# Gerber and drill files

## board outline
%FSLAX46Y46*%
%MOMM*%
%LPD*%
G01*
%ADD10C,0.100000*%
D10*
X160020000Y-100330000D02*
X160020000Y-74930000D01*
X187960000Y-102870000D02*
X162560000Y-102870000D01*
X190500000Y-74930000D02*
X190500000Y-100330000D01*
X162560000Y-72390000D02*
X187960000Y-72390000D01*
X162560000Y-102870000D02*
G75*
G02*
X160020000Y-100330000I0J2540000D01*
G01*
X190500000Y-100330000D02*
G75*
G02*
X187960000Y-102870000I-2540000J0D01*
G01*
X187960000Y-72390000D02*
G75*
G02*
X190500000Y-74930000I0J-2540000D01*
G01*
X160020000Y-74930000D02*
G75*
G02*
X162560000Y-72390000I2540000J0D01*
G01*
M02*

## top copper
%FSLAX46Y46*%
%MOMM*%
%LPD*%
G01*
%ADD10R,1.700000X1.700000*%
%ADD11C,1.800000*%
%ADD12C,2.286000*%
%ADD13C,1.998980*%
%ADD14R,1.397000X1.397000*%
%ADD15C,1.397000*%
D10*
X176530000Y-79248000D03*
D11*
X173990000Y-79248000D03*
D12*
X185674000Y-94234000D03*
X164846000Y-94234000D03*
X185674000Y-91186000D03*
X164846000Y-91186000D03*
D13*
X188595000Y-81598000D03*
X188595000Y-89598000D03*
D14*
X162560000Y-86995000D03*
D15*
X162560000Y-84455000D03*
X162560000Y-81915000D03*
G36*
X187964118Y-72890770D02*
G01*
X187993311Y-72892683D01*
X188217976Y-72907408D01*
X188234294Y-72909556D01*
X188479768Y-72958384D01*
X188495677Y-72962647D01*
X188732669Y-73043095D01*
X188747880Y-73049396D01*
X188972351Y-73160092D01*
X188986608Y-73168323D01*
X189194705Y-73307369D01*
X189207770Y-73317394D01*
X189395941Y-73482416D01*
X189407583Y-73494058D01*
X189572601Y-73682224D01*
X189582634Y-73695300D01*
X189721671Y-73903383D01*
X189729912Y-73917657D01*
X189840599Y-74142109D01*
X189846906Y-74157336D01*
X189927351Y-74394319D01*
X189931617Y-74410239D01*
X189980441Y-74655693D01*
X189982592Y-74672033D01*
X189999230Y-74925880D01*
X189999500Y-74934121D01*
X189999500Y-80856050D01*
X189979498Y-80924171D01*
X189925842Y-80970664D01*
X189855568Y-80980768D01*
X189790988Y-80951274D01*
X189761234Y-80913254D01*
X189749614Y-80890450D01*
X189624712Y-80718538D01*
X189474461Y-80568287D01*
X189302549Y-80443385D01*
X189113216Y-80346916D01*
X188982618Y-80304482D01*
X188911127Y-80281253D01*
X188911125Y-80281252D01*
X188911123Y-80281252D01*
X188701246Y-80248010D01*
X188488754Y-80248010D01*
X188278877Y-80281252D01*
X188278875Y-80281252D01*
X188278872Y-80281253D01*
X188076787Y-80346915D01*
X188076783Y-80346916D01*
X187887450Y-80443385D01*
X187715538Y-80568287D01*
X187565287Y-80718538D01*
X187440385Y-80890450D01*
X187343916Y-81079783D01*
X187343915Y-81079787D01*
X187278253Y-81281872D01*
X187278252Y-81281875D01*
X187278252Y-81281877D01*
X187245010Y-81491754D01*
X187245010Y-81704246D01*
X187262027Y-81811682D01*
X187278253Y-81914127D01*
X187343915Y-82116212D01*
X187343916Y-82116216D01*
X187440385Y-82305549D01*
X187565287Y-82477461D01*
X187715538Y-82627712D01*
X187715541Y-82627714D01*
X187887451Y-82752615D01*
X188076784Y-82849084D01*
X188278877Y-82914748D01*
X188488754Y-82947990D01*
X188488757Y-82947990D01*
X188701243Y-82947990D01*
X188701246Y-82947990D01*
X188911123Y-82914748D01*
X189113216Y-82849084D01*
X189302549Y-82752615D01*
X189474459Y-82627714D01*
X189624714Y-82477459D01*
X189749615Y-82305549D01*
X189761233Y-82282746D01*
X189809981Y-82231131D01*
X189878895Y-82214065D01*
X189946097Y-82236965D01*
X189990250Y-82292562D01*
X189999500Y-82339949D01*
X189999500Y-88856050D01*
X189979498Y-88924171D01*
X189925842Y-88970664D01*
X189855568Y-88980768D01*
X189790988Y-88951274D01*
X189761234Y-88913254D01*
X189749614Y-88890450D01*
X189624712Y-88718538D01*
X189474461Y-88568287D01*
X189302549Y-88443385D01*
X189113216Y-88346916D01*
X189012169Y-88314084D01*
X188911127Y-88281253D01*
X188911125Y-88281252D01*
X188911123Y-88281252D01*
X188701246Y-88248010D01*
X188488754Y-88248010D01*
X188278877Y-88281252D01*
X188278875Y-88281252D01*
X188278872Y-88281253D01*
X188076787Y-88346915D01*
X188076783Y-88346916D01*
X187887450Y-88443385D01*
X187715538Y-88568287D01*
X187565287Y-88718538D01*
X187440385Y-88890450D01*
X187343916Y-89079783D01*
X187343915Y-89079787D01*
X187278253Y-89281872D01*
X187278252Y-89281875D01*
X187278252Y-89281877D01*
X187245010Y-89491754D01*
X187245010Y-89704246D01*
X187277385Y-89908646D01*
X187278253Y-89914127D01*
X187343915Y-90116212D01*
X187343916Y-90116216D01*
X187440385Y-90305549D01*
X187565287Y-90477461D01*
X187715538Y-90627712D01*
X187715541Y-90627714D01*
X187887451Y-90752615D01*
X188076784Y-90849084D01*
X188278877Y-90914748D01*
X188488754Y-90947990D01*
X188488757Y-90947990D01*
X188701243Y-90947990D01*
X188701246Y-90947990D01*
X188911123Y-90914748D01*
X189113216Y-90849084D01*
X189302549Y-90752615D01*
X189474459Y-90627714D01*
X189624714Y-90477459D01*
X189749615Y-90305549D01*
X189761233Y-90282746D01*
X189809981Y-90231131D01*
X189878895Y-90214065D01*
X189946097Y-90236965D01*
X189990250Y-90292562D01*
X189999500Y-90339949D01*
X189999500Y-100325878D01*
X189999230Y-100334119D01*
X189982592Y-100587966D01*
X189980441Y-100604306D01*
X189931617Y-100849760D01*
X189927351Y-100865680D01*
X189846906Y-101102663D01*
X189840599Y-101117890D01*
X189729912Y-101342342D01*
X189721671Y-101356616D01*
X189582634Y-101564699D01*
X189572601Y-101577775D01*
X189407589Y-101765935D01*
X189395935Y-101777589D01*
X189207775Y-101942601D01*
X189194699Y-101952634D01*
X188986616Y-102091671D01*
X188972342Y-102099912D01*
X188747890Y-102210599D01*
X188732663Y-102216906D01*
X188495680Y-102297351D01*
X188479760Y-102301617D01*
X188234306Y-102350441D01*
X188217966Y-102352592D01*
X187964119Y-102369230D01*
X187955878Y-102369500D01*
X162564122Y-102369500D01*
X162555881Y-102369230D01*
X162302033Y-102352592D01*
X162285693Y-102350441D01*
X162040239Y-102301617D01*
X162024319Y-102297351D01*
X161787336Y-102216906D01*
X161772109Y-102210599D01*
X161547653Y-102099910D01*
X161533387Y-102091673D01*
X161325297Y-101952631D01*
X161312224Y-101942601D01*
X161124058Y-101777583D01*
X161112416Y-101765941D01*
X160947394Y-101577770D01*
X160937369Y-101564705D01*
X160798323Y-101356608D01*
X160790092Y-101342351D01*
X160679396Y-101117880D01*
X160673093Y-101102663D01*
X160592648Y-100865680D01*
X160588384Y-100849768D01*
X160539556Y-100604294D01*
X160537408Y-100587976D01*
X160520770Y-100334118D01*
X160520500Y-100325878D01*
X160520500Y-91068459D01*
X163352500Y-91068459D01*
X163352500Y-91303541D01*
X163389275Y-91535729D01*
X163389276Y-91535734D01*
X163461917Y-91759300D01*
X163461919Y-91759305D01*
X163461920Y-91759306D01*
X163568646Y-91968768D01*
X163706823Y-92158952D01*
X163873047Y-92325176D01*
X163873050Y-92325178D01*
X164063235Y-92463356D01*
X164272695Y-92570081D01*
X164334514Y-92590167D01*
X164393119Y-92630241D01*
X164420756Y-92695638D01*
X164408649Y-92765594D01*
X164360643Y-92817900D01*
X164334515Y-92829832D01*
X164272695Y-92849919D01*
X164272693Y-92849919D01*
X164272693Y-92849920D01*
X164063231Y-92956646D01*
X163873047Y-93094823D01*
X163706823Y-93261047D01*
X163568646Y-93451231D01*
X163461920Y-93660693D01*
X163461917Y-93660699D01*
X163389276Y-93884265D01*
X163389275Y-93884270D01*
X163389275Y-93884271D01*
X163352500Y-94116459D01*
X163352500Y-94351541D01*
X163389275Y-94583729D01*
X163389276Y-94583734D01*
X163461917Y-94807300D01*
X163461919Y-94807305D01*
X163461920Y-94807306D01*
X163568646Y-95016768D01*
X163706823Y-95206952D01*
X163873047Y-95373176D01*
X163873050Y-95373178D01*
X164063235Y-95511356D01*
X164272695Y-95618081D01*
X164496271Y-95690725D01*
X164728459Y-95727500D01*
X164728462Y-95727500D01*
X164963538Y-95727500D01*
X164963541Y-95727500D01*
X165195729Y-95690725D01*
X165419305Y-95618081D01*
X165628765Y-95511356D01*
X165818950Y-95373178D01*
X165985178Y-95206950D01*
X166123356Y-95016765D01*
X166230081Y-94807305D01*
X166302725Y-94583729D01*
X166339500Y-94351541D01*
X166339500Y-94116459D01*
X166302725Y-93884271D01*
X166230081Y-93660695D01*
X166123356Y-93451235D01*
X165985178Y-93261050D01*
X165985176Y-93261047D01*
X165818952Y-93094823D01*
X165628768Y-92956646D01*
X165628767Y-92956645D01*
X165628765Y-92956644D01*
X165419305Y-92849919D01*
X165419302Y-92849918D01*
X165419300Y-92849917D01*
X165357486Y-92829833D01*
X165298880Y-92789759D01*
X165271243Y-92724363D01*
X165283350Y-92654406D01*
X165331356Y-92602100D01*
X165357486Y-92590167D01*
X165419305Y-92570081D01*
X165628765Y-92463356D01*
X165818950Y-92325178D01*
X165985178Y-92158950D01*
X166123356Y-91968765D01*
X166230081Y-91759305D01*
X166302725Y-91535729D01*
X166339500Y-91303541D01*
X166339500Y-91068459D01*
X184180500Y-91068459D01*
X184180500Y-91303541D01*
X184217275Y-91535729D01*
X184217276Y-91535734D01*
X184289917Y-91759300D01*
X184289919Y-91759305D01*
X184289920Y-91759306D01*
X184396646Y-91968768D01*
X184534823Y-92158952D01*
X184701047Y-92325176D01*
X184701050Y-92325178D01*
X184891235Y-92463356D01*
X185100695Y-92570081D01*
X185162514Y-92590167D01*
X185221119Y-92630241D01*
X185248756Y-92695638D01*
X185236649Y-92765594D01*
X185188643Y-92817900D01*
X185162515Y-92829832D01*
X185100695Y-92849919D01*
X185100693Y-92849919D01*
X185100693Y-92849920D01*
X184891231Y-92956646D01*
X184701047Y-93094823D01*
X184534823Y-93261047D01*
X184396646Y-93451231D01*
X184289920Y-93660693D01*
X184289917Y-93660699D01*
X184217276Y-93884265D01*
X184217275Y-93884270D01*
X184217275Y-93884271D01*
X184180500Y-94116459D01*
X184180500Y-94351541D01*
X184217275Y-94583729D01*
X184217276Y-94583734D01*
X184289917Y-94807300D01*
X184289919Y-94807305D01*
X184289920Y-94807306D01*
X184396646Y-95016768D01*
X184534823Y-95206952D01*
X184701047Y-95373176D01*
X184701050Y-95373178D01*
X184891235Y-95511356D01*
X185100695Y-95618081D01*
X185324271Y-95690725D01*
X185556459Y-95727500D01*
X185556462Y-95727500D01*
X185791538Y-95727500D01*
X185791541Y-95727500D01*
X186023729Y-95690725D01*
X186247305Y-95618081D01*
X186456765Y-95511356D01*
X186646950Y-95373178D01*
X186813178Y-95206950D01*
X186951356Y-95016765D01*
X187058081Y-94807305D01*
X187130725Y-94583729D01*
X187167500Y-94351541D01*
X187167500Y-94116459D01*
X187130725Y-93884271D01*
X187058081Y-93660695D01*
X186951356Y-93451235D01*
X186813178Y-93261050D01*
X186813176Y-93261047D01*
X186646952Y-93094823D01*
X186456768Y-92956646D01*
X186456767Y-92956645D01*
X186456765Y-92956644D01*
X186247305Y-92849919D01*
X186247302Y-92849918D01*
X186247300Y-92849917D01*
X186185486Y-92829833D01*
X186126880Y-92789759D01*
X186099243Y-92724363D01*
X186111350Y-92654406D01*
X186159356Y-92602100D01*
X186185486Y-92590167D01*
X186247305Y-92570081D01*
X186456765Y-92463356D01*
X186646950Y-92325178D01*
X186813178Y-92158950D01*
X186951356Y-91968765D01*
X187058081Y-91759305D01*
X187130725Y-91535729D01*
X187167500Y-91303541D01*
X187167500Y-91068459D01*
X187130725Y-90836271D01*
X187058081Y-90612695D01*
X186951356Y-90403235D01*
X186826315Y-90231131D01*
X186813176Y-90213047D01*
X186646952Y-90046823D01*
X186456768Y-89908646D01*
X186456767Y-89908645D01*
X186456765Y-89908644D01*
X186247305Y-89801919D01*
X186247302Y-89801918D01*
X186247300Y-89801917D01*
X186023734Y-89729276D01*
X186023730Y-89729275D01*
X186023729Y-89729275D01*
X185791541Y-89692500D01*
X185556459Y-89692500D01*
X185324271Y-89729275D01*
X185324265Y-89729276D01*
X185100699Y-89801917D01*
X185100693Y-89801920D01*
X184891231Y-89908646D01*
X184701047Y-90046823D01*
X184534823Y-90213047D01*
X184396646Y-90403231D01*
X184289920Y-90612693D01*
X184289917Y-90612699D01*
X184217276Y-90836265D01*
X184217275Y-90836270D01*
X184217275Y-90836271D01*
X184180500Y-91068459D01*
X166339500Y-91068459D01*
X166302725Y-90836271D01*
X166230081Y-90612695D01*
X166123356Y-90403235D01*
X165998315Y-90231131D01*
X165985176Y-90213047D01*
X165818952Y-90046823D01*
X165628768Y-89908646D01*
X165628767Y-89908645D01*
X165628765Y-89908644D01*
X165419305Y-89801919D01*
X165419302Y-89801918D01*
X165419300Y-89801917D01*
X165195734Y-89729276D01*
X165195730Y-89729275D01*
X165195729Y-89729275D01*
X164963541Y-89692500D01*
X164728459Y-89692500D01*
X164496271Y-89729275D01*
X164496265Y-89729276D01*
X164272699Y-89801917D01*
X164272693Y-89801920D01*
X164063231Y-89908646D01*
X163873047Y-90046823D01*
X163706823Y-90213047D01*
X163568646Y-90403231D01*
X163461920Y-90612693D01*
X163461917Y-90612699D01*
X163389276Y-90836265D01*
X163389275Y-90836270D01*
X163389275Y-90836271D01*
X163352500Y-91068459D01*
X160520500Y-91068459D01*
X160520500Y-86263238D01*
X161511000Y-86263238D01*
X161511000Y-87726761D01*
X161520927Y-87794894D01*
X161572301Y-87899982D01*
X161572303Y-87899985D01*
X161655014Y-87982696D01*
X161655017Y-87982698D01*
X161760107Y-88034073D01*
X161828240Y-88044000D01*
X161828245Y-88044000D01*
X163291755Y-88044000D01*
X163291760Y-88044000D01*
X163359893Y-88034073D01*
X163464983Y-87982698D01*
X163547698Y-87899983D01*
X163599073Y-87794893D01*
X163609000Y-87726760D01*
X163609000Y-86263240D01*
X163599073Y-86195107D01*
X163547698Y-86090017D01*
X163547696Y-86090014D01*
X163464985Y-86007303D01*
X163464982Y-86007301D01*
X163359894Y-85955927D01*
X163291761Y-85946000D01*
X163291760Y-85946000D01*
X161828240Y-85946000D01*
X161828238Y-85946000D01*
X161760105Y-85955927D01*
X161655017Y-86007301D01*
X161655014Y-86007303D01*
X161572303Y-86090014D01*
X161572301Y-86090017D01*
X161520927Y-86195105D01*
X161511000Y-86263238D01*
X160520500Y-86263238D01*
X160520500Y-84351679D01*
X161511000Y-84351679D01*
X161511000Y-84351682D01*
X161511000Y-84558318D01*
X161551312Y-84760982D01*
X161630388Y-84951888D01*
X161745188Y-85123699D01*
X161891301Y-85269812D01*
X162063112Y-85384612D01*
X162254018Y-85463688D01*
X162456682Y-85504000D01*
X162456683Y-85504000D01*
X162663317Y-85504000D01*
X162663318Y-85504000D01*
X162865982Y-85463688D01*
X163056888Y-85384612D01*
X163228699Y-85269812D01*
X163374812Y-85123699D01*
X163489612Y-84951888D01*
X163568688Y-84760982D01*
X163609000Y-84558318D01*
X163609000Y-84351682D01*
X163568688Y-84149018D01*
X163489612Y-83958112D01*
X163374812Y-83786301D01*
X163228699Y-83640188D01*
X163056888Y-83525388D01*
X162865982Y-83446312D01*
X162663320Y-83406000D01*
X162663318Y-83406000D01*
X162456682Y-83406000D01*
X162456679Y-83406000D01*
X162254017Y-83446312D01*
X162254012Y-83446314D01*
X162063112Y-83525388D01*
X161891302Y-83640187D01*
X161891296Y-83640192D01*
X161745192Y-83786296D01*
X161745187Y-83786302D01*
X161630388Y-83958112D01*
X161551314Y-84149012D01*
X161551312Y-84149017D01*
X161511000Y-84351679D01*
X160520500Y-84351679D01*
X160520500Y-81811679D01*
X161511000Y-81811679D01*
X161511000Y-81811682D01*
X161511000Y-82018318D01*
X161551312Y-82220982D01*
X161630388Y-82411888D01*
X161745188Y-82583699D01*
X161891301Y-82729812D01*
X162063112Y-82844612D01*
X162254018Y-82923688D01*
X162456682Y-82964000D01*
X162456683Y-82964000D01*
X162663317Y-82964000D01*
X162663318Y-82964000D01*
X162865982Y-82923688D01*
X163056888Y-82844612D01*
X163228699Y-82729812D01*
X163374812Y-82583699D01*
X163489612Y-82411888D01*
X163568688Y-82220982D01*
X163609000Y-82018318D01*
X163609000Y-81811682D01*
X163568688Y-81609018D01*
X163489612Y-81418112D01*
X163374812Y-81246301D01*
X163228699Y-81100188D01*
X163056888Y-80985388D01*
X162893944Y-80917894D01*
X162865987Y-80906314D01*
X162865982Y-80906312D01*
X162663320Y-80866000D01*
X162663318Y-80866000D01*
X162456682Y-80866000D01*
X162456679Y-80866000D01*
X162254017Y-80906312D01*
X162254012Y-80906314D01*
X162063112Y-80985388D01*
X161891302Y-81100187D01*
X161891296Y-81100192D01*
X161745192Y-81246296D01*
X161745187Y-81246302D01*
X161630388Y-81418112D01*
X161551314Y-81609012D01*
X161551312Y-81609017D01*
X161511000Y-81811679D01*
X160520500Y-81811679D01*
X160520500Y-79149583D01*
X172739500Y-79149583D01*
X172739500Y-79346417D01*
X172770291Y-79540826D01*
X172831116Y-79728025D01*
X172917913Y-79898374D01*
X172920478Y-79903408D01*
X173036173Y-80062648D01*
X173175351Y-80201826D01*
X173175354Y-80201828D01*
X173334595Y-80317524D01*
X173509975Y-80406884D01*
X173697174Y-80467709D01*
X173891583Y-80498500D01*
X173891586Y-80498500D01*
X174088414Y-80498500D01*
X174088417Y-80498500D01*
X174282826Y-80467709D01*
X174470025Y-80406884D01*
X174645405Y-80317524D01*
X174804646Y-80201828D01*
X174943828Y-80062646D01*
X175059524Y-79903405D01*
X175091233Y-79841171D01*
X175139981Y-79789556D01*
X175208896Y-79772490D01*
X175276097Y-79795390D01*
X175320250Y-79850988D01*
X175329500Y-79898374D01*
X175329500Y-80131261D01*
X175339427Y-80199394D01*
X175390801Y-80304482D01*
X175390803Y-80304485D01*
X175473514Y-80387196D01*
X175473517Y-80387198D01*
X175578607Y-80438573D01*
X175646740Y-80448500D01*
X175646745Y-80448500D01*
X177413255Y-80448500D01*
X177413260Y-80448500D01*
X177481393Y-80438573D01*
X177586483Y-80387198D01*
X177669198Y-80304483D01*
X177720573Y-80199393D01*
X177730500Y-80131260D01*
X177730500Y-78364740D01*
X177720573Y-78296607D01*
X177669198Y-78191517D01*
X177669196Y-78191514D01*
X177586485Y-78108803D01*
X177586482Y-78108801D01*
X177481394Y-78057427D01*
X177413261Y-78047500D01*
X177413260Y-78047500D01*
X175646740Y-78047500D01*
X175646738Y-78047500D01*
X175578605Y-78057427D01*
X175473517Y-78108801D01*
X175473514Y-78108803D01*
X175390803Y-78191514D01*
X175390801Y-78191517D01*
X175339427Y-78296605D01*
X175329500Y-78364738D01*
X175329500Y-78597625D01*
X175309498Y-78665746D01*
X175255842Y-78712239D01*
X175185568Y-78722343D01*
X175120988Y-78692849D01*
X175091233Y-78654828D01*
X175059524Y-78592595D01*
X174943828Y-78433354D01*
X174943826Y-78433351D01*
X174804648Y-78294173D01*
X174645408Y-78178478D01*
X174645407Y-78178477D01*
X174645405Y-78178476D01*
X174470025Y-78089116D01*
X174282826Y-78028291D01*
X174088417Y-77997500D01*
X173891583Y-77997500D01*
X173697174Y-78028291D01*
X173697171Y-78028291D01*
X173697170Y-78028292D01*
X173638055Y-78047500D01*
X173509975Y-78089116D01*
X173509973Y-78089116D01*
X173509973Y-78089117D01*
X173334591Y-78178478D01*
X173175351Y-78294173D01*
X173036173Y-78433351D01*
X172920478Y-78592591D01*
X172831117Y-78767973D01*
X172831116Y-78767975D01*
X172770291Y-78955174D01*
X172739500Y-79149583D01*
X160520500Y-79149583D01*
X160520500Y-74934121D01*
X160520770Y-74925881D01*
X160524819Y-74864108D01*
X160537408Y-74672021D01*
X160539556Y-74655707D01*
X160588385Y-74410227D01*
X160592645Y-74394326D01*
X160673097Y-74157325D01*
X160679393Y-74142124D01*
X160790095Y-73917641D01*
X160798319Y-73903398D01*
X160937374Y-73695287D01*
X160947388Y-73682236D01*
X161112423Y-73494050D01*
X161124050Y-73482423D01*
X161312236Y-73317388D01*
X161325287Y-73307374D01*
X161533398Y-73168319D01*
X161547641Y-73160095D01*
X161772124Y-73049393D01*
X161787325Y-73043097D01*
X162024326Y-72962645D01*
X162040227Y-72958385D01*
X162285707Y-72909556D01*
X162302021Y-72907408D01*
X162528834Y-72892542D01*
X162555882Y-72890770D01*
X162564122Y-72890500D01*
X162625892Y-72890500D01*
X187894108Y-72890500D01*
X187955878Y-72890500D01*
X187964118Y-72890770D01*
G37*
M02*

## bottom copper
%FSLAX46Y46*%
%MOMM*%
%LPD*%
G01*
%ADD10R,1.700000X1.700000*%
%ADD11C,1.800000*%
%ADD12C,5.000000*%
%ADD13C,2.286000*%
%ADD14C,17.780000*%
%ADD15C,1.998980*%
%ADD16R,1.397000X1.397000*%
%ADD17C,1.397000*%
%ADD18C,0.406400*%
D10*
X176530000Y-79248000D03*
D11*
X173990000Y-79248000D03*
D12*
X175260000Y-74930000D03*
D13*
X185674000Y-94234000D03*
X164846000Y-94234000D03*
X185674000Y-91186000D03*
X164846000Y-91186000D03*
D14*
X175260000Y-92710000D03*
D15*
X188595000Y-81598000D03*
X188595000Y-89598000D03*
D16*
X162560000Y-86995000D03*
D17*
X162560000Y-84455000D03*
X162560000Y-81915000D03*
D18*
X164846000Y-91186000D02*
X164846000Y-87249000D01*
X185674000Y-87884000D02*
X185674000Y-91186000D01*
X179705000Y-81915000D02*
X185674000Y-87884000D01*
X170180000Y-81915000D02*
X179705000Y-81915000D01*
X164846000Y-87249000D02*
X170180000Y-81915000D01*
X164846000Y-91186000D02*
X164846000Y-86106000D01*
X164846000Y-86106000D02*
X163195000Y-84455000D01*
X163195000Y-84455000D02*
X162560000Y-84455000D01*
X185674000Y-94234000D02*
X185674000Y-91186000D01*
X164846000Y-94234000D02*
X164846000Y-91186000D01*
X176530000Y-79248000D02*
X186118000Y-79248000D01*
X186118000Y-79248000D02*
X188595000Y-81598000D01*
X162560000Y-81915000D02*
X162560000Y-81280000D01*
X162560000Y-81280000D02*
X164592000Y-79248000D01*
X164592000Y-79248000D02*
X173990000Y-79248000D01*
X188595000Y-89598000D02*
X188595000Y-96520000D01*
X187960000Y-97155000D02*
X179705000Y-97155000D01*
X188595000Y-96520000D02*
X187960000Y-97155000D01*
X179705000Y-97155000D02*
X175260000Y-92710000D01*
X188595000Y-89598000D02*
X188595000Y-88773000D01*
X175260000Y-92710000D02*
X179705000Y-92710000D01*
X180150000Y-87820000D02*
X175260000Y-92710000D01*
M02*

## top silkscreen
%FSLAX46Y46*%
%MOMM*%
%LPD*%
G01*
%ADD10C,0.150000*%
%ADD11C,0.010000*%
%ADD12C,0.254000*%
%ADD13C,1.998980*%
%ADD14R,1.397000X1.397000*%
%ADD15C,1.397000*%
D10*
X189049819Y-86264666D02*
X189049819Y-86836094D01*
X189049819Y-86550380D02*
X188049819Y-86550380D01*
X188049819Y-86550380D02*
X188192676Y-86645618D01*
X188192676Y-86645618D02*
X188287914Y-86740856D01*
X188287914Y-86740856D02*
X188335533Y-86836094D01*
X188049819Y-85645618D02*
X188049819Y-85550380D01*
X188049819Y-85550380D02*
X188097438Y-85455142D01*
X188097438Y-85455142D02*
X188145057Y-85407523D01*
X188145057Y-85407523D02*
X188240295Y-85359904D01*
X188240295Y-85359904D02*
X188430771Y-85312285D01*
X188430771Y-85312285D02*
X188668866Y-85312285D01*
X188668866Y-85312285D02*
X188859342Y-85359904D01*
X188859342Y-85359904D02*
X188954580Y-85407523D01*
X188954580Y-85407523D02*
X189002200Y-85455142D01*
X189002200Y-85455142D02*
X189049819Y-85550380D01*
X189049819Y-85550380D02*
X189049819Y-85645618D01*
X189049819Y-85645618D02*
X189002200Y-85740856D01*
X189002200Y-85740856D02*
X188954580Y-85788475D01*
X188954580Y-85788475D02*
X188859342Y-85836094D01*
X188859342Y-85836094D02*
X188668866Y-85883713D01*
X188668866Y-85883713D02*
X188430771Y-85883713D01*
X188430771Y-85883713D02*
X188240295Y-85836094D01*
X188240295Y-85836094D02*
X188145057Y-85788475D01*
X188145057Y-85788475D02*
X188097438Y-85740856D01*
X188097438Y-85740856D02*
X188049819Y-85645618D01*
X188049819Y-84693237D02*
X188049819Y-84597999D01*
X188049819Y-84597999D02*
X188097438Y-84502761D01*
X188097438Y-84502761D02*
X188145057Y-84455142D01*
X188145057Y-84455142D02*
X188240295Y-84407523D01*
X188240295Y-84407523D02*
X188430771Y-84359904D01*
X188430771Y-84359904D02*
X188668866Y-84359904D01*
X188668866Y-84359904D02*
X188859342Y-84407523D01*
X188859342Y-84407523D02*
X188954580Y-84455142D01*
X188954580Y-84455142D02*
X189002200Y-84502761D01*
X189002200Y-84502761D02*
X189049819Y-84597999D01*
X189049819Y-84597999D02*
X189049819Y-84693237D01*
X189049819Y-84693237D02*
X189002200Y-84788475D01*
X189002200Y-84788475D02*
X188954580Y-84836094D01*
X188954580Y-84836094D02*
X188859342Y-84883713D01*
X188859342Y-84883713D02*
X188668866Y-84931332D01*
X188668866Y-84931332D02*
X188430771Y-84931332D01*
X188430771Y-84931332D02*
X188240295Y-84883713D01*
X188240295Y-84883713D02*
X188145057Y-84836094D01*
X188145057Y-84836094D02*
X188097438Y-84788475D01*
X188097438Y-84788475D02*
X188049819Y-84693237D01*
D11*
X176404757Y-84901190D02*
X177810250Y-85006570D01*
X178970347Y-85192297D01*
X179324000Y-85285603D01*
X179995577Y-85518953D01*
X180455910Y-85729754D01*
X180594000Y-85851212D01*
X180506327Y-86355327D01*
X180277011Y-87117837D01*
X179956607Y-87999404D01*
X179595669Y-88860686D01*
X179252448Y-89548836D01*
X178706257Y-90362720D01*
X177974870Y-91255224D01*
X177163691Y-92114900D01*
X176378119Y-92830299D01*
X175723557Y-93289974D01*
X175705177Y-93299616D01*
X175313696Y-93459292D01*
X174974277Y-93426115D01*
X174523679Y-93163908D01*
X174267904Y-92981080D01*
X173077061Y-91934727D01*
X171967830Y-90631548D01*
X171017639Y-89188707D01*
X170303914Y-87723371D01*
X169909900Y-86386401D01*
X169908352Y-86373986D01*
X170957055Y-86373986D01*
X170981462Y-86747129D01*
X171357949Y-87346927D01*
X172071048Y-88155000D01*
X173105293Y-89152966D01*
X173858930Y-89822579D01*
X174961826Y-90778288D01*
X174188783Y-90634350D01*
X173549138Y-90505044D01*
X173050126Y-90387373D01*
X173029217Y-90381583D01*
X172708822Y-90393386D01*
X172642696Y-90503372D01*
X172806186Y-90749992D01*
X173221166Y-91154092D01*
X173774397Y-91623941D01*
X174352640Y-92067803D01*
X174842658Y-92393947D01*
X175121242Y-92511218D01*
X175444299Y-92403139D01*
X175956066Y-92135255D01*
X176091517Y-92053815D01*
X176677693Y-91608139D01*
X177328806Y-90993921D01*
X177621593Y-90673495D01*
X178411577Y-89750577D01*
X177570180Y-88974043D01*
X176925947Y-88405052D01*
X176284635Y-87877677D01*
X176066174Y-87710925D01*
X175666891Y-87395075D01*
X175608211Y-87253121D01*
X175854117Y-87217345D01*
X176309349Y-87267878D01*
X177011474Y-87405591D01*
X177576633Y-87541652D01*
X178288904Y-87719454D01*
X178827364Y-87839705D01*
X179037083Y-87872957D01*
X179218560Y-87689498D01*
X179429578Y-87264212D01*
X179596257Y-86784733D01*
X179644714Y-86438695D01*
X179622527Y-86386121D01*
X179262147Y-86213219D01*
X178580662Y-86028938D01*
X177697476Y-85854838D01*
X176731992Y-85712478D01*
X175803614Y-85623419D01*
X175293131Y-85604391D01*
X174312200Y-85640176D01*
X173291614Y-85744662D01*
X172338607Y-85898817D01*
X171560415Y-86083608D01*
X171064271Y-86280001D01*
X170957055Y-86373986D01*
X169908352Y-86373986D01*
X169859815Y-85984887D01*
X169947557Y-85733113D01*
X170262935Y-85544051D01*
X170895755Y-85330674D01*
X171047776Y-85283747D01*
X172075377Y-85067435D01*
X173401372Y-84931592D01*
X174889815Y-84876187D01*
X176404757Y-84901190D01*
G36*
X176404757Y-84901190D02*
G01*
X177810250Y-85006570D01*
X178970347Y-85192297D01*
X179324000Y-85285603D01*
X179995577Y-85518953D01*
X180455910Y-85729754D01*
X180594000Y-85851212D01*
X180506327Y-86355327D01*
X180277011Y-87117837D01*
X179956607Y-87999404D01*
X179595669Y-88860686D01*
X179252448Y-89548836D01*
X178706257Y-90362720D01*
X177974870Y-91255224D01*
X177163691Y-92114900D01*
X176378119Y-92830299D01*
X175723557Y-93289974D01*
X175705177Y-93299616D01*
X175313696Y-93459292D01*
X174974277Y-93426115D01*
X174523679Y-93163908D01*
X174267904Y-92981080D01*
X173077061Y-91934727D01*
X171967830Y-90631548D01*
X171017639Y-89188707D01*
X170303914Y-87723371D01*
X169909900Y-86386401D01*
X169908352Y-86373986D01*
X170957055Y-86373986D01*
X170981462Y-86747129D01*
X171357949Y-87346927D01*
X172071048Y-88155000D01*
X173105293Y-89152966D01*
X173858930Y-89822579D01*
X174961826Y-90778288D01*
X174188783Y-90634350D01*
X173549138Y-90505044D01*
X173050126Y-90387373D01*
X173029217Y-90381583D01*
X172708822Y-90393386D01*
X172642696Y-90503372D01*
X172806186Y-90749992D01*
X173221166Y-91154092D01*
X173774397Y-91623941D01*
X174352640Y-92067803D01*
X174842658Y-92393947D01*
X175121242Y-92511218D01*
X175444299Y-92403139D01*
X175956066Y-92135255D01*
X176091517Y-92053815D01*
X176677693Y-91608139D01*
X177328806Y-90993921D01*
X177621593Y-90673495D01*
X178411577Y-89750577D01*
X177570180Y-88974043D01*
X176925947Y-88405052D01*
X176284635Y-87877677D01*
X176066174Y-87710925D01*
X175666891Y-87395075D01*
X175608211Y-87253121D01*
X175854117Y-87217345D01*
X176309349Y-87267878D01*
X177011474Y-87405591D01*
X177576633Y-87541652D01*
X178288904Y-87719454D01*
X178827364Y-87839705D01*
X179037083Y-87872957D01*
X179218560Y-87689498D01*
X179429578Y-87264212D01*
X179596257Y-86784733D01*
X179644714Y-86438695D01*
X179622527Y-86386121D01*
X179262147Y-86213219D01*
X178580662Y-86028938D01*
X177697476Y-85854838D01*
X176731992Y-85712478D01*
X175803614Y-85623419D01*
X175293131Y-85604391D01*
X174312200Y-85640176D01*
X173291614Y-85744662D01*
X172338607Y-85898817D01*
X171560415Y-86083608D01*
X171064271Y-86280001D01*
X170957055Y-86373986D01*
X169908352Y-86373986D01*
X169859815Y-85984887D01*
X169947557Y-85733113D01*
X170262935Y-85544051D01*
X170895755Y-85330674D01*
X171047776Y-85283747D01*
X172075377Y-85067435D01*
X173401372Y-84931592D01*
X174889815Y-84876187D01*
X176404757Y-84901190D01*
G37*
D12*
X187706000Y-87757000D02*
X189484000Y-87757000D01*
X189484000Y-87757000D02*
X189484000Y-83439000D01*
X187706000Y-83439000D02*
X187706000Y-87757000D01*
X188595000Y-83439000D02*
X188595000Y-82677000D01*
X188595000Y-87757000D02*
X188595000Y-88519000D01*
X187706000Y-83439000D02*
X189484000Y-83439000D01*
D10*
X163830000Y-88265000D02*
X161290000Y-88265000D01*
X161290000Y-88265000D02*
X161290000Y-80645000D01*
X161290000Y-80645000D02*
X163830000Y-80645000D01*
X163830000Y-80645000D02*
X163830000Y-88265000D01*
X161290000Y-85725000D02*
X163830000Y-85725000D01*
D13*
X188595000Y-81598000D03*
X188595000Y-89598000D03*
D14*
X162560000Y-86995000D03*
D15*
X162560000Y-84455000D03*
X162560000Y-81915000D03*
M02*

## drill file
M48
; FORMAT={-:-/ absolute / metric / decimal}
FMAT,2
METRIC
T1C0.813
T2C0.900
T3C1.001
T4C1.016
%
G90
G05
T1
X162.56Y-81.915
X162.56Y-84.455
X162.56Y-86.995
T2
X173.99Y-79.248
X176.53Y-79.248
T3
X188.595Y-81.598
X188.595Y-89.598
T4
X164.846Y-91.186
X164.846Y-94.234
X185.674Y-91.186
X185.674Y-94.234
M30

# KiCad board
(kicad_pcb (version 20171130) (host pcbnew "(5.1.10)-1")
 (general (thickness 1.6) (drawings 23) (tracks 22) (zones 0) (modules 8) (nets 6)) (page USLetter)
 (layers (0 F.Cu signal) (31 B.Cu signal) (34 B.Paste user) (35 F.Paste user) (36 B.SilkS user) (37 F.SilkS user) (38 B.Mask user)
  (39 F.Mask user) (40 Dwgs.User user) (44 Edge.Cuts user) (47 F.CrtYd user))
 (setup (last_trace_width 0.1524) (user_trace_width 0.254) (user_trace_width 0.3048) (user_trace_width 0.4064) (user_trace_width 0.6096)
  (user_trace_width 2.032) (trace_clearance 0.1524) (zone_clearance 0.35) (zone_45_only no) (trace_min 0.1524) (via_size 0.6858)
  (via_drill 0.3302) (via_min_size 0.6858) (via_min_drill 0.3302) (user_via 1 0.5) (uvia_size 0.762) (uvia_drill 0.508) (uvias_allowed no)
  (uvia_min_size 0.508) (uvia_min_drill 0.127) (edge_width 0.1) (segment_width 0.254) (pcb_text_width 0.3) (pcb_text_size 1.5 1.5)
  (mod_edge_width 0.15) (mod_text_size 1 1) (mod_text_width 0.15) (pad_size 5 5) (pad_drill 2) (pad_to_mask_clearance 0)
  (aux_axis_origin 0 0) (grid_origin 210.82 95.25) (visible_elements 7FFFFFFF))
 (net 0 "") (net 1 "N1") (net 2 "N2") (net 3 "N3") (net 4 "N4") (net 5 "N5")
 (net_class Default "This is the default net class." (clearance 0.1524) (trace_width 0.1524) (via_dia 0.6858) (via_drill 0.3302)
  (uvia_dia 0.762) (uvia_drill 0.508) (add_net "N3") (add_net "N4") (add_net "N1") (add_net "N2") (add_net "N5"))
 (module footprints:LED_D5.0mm (layer F.Cu) (at 176.53 79.248 180)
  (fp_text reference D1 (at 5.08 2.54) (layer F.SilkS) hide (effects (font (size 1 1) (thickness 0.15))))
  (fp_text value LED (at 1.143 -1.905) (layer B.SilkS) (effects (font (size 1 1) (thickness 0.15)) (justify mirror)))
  (pad 1 thru_hole rect (at 0 0 180) (size 1.7 1.7) (drill 0.9) (layers B.Cu B.Mask) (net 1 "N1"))
  (pad 2 thru_hole circle (at 2.54 0 180) (size 1.8 1.8) (drill 0.9) (layers B.Cu B.Mask) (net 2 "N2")))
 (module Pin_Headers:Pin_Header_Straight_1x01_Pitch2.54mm (layer F.Cu) (at 175.26 74.93)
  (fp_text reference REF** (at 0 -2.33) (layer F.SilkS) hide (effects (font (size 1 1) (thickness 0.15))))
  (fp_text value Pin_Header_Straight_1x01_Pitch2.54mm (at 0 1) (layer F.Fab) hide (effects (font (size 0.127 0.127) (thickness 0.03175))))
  (pad 1 smd circle (at 0 0) (size 5 5) (layers B.Cu B.Paste B.Mask)))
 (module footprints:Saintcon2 (layer F.Cu) (at 175.514 86.106)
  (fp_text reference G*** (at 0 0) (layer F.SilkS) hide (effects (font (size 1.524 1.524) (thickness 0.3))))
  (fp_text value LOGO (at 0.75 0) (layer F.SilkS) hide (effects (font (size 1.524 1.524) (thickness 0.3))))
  (fp_poly
   (pts (xy 0.890757 -1.20481) (xy 2.29625 -1.09943) (xy 3.456347 -0.913703) (xy 3.81 -0.820397) (xy 4.481577 -0.587047)
    (xy 4.94191 -0.376246) (xy 5.08 -0.254788) (xy 4.992327 0.249327) (xy 4.763011 1.011837) (xy 4.442607 1.893404) (xy 4.081669 2.754686)
    (xy 3.738448 3.442836) (xy 3.192257 4.25672) (xy 2.46087 5.149224) (xy 1.649691 6.0089) (xy 0.864119 6.724299) (xy 0.209557 7.183974)
    (xy 0.191177 7.193616) (xy -0.200304 7.353292) (xy -0.539723 7.320115) (xy -0.990321 7.057908) (xy -1.246096 6.87508)
    (xy -2.436939 5.828727) (xy -3.54617 4.525548) (xy -4.496361 3.082707) (xy -5.210086 1.617371) (xy -5.6041 0.280401)
    (xy -5.605648 0.267986) (xy -4.556945 0.267986) (xy -4.532538 0.641129) (xy -4.156051 1.240927) (xy -3.442952 2.049)
    (xy -2.408707 3.046966) (xy -1.65507 3.716579) (xy -0.552174 4.672288) (xy -1.325217 4.52835) (xy -1.964862 4.399044)
    (xy -2.463874 4.281373) (xy -2.484783 4.275583) (xy -2.805178 4.287386) (xy -2.871304 4.397372) (xy -2.707814 4.643992)
    (xy -2.292834 5.048092) (xy -1.739603 5.517941) (xy -1.16136 5.961803) (xy -0.671342 6.287947) (xy -0.392758 6.405218)
    (xy -0.069701 6.297139) (xy 0.442066 6.029255) (xy 0.577517 5.947815) (xy 1.163693 5.502139) (xy 1.814806 4.887921)
    (xy 2.107593 4.567495) (xy 2.897577 3.644577) (xy 2.05618 2.868043) (xy 1.411947 2.299052) (xy 0.770635 1.771677) (xy 0.552174 1.604925)
    (xy 0.152891 1.289075) (xy 0.094211 1.147121) (xy 0.340117 1.111345) (xy 0.795349 1.161878) (xy 1.497474 1.299591)
    (xy 2.062633 1.435652) (xy 2.774904 1.613454) (xy 3.313364 1.733705) (xy 3.523083 1.766957) (xy 3.70456 1.583498) (xy 3.915578 1.158212)
    (xy 4.082257 0.678733) (xy 4.130714 0.332695) (xy 4.108527 0.280121) (xy 3.748147 0.107219) (xy 3.066662 -0.077062)
    (xy 2.183476 -0.251162) (xy 1.217992 -0.393522) (xy 0.289614 -0.482581) (xy -0.220869 -0.501609) (xy -1.2018 -0.465824)
    (xy -2.222386 -0.361338) (xy -3.175393 -0.207183) (xy -3.953585 -0.022392) (xy -4.449729 0.174001) (xy -4.556945 0.267986)
    (xy -5.605648 0.267986) (xy -5.654185 -0.121113) (xy -5.566443 -0.372887) (xy -5.251065 -0.561949) (xy -4.618245 -0.775326)
    (xy -4.466224 -0.822253) (xy -3.438623 -1.038565) (xy -2.112628 -1.174408) (xy -0.624185 -1.229813) (xy 0.890757 -1.20481))
   (layer F.SilkS) (width 0.01)))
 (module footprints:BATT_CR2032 (layer B.Cu) (at 175.26 92.71 180)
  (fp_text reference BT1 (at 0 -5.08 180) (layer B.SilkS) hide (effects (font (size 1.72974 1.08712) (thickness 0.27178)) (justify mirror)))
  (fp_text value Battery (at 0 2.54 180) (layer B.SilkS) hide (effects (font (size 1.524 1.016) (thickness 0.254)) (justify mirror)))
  (pad 1 thru_hole circle (at -10.414 -1.524 180) (size 2.286 2.286) (drill 1.016) (layers *.Cu *.Mask B.SilkS) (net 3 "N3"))
  (pad 1 thru_hole circle (at 10.414 -1.524 180) (size 2.286 2.286) (drill 1.016) (layers *.Cu *.Mask B.SilkS) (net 3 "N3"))
  (pad 1 thru_hole circle (at -10.414 1.524 180) (size 2.286 2.286) (drill 1.016) (layers *.Cu *.Mask B.SilkS) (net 3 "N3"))
  (pad 1 thru_hole circle (at 10.414 1.524 180) (size 2.286 2.286) (drill 1.016) (layers *.Cu *.Mask B.SilkS) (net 3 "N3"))
  (pad 2 smd circle (at 0 0 180) (size 17.78 17.78) (layers B.Cu B.Paste B.Mask) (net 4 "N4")))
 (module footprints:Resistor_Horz (layer F.Cu) (at 188.595 85.598 270)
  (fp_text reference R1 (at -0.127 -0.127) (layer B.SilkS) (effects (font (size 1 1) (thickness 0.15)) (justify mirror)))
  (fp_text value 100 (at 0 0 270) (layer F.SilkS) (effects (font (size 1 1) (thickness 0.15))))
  (fp_line (start 2.159 0.889) (end 2.159 -0.889) (layer F.SilkS) (width 0.254))
  (fp_line (start 2.159 -0.889) (end -2.159 -0.889) (layer F.SilkS) (width 0.254))
  (fp_line (start -2.159 0.889) (end 2.159 0.889) (layer F.SilkS) (width 0.254))
  (fp_line (start -2.159 0) (end -2.921 0) (layer F.SilkS) (width 0.254))
  (fp_line (start 2.159 0) (end 2.921 0) (layer F.SilkS) (width 0.254))
  (fp_line (start -2.159 0.889) (end -2.159 -0.889) (layer F.SilkS) (width 0.254))
  (pad 1 thru_hole circle (at -4 0 270) (size 1.99898 1.99898) (drill 1.00076) (layers *.Cu *.SilkS *.Mask) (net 1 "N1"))
  (pad 2 thru_hole circle (at 4 0 270) (size 1.99898 1.99898) (drill 1.00076) (layers *.Cu *.SilkS *.Mask) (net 4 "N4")))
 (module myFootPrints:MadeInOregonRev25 (layer F.Cu) (at 167.64 76.454)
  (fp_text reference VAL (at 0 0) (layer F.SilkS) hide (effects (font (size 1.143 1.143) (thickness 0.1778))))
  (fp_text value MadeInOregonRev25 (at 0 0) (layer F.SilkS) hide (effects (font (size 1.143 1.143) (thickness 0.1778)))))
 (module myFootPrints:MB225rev (layer F.Cu) (at 184.15 76.2)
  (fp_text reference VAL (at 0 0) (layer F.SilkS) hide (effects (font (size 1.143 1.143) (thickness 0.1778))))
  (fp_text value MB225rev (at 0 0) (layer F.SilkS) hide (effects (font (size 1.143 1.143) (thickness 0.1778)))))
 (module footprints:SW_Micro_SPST (layer F.Cu) (at 162.56 84.455 90)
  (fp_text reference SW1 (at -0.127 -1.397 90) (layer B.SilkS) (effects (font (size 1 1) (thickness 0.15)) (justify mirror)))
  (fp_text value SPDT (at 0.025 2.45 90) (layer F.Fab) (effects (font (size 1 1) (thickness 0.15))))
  (fp_line (start -3.81 1.27) (end -3.81 -1.27) (layer F.SilkS) (width 0.15))
  (fp_line (start -3.81 -1.27) (end 3.81 -1.27) (layer F.SilkS) (width 0.15))
  (fp_line (start 3.81 -1.27) (end 3.81 1.27) (layer F.SilkS) (width 0.15))
  (fp_line (start 3.81 1.27) (end -3.81 1.27) (layer F.SilkS) (width 0.15))
  (fp_line (start -1.27 -1.27) (end -1.27 1.27) (layer F.SilkS) (width 0.15))
  (pad 1 thru_hole rect (at -2.54 0 90) (size 1.397 1.397) (drill 0.8128) (layers *.Cu *.Mask F.SilkS) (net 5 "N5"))
  (pad 2 thru_hole circle (at 0 0 90) (size 1.397 1.397) (drill 0.8128) (layers *.Cu *.Mask F.SilkS) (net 3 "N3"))
  (pad 3 thru_hole circle (at 2.54 0 90) (size 1.397 1.397) (drill 0.8128) (layers *.Cu *.Mask F.SilkS) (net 2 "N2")))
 (gr_line (start 160.02 100.33) (end 160.02 74.93) (angle 90) (layer Edge.Cuts) (width 0.1))
 (gr_line (start 187.96 102.87) (end 162.56 102.87) (angle 90) (layer Edge.Cuts) (width 0.1))
 (gr_line (start 190.5 74.93) (end 190.5 100.33) (angle 90) (layer Edge.Cuts) (width 0.1))
 (gr_line (start 162.56 72.39) (end 187.96 72.39) (angle 90) (layer Edge.Cuts) (width 0.1))
 (gr_arc (start 162.56 100.33) (end 162.56 102.87) (angle 90) (layer Edge.Cuts) (width 0.1))
 (gr_arc (start 187.96 100.33) (end 190.5 100.33) (angle 90) (layer Edge.Cuts) (width 0.1))
 (gr_arc (start 187.96 74.93) (end 187.96 72.39) (angle 90) (layer Edge.Cuts) (width 0.1))
 (gr_arc (start 162.56 74.93) (end 160.02 74.93) (angle 90) (layer Edge.Cuts) (width 0.1))
 (segment (start 164.846 91.186) (end 164.846 87.249) (width 0.4064) (layer B.Cu) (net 3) (status 10))
 (segment (start 185.674 87.884) (end 185.674 91.186) (width 0.4064) (layer B.Cu) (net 3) (status 20))
 (segment (start 179.705 81.915) (end 185.674 87.884) (width 0.4064) (layer B.Cu) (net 3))
 (segment (start 170.18 81.915) (end 179.705 81.915) (width 0.4064) (layer B.Cu) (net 3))
 (segment (start 164.846 87.249) (end 170.18 81.915) (width 0.4064) (layer B.Cu) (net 3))
 (segment (start 164.846 91.186) (end 164.846 86.106) (width 0.4064) (layer B.Cu) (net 3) (status 10))
 (segment (start 164.846 86.106) (end 163.195 84.455) (width 0.4064) (layer B.Cu) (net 3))
 (segment (start 163.195 84.455) (end 162.56 84.455) (width 0.4064) (layer B.Cu) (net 3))
 (segment (start 185.674 94.234) (end 185.674 91.186) (width 0.4064) (layer B.Cu) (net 3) (status 30))
 (segment (start 164.846 94.234) (end 164.846 91.186) (width 0.4064) (layer B.Cu) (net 3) (status 30))
 (segment (start 176.53 79.248) (end 186.118 79.248) (width 0.4064) (layer B.Cu) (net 1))
 (segment (start 186.118 79.248) (end 188.595 81.598) (width 0.4064) (layer B.Cu) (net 1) (status 20))
 (segment (start 162.56 81.915) (end 162.56 81.28) (width 0.4064) (layer B.Cu) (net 2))
 (segment (start 162.56 81.28) (end 164.592 79.248) (width 0.4064) (layer B.Cu) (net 2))
 (segment (start 164.592 79.248) (end 173.99 79.248) (width 0.4064) (layer B.Cu) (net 2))
 (segment (start 188.595 89.598) (end 188.595 96.52) (width 0.4064) (layer B.Cu) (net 4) (status 10))
 (segment (start 187.96 97.155) (end 179.705 97.155) (width 0.4064) (layer B.Cu) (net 4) (status 20))
 (segment (start 188.595 96.52) (end 187.96 97.155) (width 0.4064) (layer B.Cu) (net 4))
 (segment (start 179.705 97.155) (end 175.26 92.71) (width 0.4064) (layer B.Cu) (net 4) (status 30))
 (segment (start 188.595 89.598) (end 188.595 88.773) (width 0.4064) (layer B.Cu) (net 4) (status 30))
 (segment (start 175.26 92.71) (end 179.705 92.71) (width 0.4064) (layer B.Cu) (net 4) (status 30))
 (segment (start 180.15 87.82) (end 175.26 92.71) (width 0.4064) (layer B.Cu) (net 4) (status 30))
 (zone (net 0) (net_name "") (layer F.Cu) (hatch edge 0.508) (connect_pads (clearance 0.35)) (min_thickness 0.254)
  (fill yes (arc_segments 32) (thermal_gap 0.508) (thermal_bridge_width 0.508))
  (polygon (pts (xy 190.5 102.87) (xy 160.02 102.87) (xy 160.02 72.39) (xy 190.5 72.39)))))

